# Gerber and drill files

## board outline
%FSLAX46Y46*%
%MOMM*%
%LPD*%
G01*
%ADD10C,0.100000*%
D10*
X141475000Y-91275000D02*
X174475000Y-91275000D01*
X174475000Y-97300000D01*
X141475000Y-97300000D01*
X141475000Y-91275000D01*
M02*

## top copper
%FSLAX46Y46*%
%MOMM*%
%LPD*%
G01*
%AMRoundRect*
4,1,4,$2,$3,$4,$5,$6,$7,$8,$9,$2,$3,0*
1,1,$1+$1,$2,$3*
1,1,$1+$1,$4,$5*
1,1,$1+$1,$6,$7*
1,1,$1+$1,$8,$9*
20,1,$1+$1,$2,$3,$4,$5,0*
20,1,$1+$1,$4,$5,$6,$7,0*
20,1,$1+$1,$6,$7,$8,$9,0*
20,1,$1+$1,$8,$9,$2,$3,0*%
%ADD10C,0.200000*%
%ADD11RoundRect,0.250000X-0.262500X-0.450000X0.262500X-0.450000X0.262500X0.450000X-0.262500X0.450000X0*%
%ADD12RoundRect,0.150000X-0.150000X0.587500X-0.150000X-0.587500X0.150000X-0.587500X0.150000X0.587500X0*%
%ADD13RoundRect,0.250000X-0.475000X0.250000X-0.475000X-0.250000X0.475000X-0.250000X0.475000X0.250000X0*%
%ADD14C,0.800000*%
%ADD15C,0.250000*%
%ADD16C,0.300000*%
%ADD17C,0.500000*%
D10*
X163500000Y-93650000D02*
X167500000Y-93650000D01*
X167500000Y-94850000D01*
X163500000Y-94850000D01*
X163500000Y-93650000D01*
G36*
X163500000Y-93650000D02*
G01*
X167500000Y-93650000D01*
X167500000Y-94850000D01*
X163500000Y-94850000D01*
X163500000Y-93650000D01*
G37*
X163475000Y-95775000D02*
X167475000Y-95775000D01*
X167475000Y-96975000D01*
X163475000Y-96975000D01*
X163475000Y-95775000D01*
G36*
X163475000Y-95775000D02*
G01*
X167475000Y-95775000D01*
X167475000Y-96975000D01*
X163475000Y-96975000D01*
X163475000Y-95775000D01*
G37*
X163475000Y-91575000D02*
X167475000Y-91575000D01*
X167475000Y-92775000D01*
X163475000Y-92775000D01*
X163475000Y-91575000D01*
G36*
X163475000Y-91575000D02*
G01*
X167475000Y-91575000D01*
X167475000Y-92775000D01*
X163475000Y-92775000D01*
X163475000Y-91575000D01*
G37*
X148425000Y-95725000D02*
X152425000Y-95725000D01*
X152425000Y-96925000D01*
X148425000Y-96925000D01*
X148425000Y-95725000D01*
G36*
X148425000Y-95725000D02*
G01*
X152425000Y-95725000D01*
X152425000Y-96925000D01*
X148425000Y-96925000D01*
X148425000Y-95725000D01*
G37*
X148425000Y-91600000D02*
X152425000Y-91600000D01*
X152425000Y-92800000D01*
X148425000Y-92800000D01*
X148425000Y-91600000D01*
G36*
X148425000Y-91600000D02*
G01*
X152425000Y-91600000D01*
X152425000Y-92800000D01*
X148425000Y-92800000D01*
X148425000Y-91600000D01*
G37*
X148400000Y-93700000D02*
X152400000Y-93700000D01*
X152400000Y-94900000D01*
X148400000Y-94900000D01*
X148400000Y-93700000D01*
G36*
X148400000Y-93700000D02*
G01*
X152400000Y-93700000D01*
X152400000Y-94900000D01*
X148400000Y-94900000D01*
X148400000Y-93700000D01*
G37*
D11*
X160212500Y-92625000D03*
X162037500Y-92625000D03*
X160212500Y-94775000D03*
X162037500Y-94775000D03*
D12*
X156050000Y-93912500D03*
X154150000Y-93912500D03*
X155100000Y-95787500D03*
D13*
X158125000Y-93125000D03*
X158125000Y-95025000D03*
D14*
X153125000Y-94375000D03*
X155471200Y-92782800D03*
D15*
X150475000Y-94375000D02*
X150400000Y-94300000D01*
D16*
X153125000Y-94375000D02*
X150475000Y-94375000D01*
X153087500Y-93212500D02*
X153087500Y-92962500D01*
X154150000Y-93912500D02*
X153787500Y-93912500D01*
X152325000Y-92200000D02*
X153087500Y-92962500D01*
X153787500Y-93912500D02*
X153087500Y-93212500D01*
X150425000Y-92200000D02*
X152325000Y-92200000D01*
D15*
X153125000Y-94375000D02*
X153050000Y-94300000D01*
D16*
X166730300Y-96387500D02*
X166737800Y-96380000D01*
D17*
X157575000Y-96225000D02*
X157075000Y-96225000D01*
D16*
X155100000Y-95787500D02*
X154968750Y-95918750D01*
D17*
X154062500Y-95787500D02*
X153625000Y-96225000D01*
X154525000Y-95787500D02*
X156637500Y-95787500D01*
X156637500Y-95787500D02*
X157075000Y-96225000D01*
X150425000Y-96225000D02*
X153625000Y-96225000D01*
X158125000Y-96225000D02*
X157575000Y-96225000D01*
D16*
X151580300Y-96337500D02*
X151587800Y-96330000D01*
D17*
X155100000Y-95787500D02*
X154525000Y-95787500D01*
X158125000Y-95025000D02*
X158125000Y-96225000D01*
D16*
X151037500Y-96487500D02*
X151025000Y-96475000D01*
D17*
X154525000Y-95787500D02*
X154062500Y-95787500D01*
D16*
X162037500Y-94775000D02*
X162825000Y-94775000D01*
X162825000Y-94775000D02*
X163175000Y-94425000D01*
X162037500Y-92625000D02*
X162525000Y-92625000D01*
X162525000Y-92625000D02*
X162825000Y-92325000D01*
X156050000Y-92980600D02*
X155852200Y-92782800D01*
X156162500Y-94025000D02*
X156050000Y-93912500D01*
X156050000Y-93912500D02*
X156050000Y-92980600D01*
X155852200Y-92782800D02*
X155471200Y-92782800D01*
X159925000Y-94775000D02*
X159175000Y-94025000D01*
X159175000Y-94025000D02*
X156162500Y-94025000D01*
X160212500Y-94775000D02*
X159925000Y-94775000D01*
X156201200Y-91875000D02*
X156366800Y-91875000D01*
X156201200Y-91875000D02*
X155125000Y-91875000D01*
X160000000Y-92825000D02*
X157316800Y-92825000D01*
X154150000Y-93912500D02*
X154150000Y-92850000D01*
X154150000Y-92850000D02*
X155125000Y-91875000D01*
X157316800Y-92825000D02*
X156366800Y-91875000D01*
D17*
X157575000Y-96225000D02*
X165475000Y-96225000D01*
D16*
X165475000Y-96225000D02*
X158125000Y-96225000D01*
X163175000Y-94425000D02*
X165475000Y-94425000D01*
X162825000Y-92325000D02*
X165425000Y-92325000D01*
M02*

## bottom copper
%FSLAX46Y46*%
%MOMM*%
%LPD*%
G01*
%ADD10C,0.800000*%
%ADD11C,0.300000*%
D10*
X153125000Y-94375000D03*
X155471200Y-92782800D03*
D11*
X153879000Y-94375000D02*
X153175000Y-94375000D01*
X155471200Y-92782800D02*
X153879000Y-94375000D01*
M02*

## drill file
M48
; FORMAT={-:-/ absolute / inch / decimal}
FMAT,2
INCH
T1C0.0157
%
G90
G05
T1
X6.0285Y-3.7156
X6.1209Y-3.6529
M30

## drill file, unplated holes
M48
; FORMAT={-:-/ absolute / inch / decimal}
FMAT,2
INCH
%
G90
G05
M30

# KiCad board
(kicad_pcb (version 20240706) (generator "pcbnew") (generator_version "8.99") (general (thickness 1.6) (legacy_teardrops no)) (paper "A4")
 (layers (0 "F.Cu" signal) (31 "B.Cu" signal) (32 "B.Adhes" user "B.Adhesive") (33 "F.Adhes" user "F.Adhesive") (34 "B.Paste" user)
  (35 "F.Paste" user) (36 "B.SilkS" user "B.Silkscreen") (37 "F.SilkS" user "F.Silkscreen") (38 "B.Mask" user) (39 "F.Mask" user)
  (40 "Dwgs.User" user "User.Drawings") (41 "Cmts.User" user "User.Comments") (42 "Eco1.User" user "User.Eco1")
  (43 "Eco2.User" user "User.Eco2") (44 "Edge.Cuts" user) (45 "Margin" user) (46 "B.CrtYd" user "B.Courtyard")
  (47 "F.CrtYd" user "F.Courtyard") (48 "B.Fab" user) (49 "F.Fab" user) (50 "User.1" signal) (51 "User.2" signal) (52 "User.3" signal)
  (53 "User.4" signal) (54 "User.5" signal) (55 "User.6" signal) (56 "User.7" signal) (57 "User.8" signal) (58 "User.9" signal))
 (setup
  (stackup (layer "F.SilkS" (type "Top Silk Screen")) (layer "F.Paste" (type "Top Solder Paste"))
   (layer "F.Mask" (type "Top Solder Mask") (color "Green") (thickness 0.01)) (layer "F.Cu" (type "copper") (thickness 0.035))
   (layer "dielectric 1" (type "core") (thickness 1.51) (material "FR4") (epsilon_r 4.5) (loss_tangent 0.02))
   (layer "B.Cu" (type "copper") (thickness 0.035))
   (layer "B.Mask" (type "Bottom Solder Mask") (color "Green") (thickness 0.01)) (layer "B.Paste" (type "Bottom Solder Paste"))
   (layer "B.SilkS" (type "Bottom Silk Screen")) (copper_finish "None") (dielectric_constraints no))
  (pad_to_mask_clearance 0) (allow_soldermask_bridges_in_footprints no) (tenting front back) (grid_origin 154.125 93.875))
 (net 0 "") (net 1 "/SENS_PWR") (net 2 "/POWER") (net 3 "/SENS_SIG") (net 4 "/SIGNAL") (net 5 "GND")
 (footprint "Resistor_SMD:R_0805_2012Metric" (layer "F.Cu") (at 161.125 92.625)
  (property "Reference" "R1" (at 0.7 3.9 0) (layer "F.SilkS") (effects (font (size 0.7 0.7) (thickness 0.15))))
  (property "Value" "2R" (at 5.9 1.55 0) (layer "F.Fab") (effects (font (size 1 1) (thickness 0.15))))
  (pad "1" smd roundrect (at -0.9125 0) (size 1.025 1.4) (layers "F.Cu" "F.Paste" "F.Mask") (roundrect_rratio 0.243902) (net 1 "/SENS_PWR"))
  (pad "2" smd roundrect (at 0.9125 0) (size 1.025 1.4) (layers "F.Cu" "F.Paste" "F.Mask") (roundrect_rratio 0.243902) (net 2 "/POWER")))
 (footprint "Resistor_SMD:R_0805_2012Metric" (layer "F.Cu") (at 161.125 94.775)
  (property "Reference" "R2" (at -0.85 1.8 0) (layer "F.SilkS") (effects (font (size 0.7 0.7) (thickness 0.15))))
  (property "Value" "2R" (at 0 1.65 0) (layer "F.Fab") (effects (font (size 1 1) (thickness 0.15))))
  (pad "1" smd roundrect (at -0.9125 0) (size 1.025 1.4) (layers "F.Cu" "F.Paste" "F.Mask") (roundrect_rratio 0.243902) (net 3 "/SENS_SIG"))
  (pad "2" smd roundrect (at 0.9125 0) (size 1.025 1.4) (layers "F.Cu" "F.Paste" "F.Mask") (roundrect_rratio 0.243902) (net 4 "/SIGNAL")))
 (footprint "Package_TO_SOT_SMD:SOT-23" (layer "F.Cu") (at 155.1 94.85 -90)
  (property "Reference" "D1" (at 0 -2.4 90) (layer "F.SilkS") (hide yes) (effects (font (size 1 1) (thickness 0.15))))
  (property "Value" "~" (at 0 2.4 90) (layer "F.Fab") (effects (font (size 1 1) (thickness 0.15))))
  (pad "1" smd roundrect (at -0.9375 -0.95 270) (size 1.475 0.6) (layers "F.Cu" "F.Paste" "F.Mask") (roundrect_rratio 0.25)
   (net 3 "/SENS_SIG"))
  (pad "2" smd roundrect (at -0.9375 0.95 270) (size 1.475 0.6) (layers "F.Cu" "F.Paste" "F.Mask") (roundrect_rratio 0.25)
   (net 1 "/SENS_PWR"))
  (pad "3" smd roundrect (at 0.9375 0 270) (size 1.475 0.6) (layers "F.Cu" "F.Paste" "F.Mask") (roundrect_rratio 0.25) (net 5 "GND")))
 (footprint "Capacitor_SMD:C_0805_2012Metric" (layer "F.Cu") (at 158.125 94.075 -90)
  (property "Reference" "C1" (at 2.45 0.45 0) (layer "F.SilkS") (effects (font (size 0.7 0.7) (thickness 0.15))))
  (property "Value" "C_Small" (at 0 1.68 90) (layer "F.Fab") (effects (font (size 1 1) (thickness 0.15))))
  (pad "1" smd roundrect (at -0.95 0 270) (size 1 1.45) (layers "F.Cu" "F.Paste" "F.Mask") (roundrect_rratio 0.25) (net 1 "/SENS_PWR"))
  (pad "2" smd roundrect (at 0.95 0 270) (size 1 1.45) (layers "F.Cu" "F.Paste" "F.Mask") (roundrect_rratio 0.25) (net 5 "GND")))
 (gr_rect (start 148.425 91.6) (end 152.425 92.8) (stroke (width 0.2) (type solid)) (fill solid) (layer "F.Cu") (net 1))
 (gr_rect (start 148.425 95.725) (end 152.425 96.925) (stroke (width 0.2) (type solid)) (fill solid) (layer "F.Cu") (net 5))
 (gr_rect (start 163.475 91.575) (end 167.475 92.775) (stroke (width 0.2) (type solid)) (fill solid) (layer "F.Cu") (net 2))
 (gr_rect (start 163.5 93.65) (end 167.5 94.85) (stroke (width 0.2) (type solid)) (fill solid) (layer "F.Cu") (net 4))
 (gr_rect (start 163.475 95.775) (end 167.475 96.975) (stroke (width 0.2) (type solid)) (fill solid) (layer "F.Cu") (net 5))
 (gr_rect (start 148.4 93.7) (end 152.4 94.9) (stroke (width 0.2) (type solid)) (fill solid) (layer "F.Cu") (net 3))
 (gr_rect (start 141.475 91.275) (end 174.475 97.3) (stroke (width 0.1) (type solid)) (fill none) (layer "Edge.Cuts"))
 (segment (start 157.575 96.225) (end 157.075 96.225) (width 0.5) (layer "F.Cu") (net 5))
 (segment (start 155.1 95.7875) (end 154.96875 95.91875) (width 0.3) (layer "F.Cu") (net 5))
 (segment (start 154.0625 95.7875) (end 153.625 96.225) (width 0.5) (layer "F.Cu") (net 5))
 (segment (start 154.525 95.7875) (end 156.6375 95.7875) (width 0.5) (layer "F.Cu") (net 5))
 (segment (start 156.6375 95.7875) (end 157.075 96.225) (width 0.5) (layer "F.Cu") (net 5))
 (segment (start 157.575 96.225) (end 165.475 96.225) (width 0.5) (layer "F.Cu") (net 5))
 (segment (start 166.7303 96.3875) (end 166.7378 96.38) (width 0.3) (layer "F.Cu") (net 5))
 (segment (start 150.425 96.225) (end 153.625 96.225) (width 0.5) (layer "F.Cu") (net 5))
 (segment (start 158.125 96.225) (end 157.575 96.225) (width 0.5) (layer "F.Cu") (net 5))
 (segment (start 151.5803 96.3375) (end 151.5878 96.33) (width 0.3) (layer "F.Cu") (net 5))
 (segment (start 155.1 95.7875) (end 154.525 95.7875) (width 0.5) (layer "F.Cu") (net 5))
 (segment (start 158.125 95.025) (end 158.125 96.225) (width 0.5) (layer "F.Cu") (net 5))
 (segment (start 151.0375 96.4875) (end 151.025 96.475) (width 0.3) (layer "F.Cu") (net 5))
 (segment (start 165.475 96.225) (end 158.125 96.225) (width 0.3) (layer "F.Cu") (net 5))
 (segment (start 154.525 95.7875) (end 154.0625 95.7875) (width 0.5) (layer "F.Cu") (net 5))
 (segment (start 162.0375 94.775) (end 162.825 94.775) (width 0.3) (layer "F.Cu") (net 4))
 (segment (start 162.825 94.775) (end 163.175 94.425) (width 0.3) (locked yes) (layer "F.Cu") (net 4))
 (segment (start 163.175 94.425) (end 165.475 94.425) (width 0.3) (layer "F.Cu") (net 4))
 (segment (start 162.825 92.325) (end 165.425 92.325) (width 0.3) (layer "F.Cu") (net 2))
 (segment (start 162.0375 92.625) (end 162.525 92.625) (width 0.3) (layer "F.Cu") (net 2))
 (segment (start 162.525 92.625) (end 162.825 92.325) (width 0.3) (layer "F.Cu") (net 2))
 (segment (start 156.2012 91.875) (end 156.3668 91.875) (width 0.3) (layer "F.Cu") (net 1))
 (segment (start 152.325 92.2) (end 153.0875 92.9625) (width 0.3) (layer "F.Cu") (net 1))
 (segment (start 156.2012 91.875) (end 155.125 91.875) (width 0.3) (layer "F.Cu") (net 1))
 (segment (start 154.15 93.9125) (end 153.7875 93.9125) (width 0.3) (layer "F.Cu") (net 1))
 (segment (start 160 92.825) (end 157.3168 92.825) (width 0.3) (layer "F.Cu") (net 1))
 (segment (start 153.7875 93.9125) (end 153.0875 93.2125) (width 0.3) (layer "F.Cu") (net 1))
 (segment (start 154.15 93.9125) (end 154.15 92.85) (width 0.3) (layer "F.Cu") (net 1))
 (segment (start 154.15 92.85) (end 155.125 91.875) (width 0.3) (layer "F.Cu") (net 1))
 (segment (start 157.3168 92.825) (end 156.3668 91.875) (width 0.3) (layer "F.Cu") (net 1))
 (segment (start 150.425 92.2) (end 152.325 92.2) (width 0.3) (layer "F.Cu") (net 1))
 (segment (start 153.0875 93.2125) (end 153.0875 92.9625) (width 0.3) (layer "F.Cu") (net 1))
 (segment (start 153.125 94.375) (end 150.475 94.375) (width 0.3) (layer "F.Cu") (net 3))
 (segment (start 156.05 92.9806) (end 155.8522 92.7828) (width 0.3) (layer "F.Cu") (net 3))
 (segment (start 156.1625 94.025) (end 156.05 93.9125) (width 0.3) (layer "F.Cu") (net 3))
 (segment (start 156.05 93.9125) (end 156.05 92.9806) (width 0.3) (layer "F.Cu") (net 3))
 (segment (start 155.8522 92.7828) (end 155.4712 92.7828) (width 0.3) (layer "F.Cu") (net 3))
 (segment (start 159.925 94.775) (end 159.175 94.025) (width 0.3) (layer "F.Cu") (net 3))
 (segment (start 159.175 94.025) (end 156.1625 94.025) (width 0.3) (layer "F.Cu") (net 3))
 (segment (start 153.125 94.375) (end 153.05 94.3) (width 0.25) (layer "F.Cu") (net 3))
 (segment (start 160.2125 94.775) (end 159.925 94.775) (width 0.3) (layer "F.Cu") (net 3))
 (segment (start 150.475 94.375) (end 150.4 94.3) (width 0.25) (layer "F.Cu") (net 3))
 (via (at 155.4712 92.7828) (size 0.8) (drill 0.4) (layers "F.Cu" "B.Cu") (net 3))
 (via (at 153.125 94.375) (size 0.8) (drill 0.4) (layers "F.Cu" "B.Cu") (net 3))
 (segment (start 155.4712 92.7828) (end 153.879 94.375) (width 0.3) (layer "B.Cu") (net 3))
 (segment (start 153.879 94.375) (end 153.175 94.375) (width 0.3) (layer "B.Cu") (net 3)))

